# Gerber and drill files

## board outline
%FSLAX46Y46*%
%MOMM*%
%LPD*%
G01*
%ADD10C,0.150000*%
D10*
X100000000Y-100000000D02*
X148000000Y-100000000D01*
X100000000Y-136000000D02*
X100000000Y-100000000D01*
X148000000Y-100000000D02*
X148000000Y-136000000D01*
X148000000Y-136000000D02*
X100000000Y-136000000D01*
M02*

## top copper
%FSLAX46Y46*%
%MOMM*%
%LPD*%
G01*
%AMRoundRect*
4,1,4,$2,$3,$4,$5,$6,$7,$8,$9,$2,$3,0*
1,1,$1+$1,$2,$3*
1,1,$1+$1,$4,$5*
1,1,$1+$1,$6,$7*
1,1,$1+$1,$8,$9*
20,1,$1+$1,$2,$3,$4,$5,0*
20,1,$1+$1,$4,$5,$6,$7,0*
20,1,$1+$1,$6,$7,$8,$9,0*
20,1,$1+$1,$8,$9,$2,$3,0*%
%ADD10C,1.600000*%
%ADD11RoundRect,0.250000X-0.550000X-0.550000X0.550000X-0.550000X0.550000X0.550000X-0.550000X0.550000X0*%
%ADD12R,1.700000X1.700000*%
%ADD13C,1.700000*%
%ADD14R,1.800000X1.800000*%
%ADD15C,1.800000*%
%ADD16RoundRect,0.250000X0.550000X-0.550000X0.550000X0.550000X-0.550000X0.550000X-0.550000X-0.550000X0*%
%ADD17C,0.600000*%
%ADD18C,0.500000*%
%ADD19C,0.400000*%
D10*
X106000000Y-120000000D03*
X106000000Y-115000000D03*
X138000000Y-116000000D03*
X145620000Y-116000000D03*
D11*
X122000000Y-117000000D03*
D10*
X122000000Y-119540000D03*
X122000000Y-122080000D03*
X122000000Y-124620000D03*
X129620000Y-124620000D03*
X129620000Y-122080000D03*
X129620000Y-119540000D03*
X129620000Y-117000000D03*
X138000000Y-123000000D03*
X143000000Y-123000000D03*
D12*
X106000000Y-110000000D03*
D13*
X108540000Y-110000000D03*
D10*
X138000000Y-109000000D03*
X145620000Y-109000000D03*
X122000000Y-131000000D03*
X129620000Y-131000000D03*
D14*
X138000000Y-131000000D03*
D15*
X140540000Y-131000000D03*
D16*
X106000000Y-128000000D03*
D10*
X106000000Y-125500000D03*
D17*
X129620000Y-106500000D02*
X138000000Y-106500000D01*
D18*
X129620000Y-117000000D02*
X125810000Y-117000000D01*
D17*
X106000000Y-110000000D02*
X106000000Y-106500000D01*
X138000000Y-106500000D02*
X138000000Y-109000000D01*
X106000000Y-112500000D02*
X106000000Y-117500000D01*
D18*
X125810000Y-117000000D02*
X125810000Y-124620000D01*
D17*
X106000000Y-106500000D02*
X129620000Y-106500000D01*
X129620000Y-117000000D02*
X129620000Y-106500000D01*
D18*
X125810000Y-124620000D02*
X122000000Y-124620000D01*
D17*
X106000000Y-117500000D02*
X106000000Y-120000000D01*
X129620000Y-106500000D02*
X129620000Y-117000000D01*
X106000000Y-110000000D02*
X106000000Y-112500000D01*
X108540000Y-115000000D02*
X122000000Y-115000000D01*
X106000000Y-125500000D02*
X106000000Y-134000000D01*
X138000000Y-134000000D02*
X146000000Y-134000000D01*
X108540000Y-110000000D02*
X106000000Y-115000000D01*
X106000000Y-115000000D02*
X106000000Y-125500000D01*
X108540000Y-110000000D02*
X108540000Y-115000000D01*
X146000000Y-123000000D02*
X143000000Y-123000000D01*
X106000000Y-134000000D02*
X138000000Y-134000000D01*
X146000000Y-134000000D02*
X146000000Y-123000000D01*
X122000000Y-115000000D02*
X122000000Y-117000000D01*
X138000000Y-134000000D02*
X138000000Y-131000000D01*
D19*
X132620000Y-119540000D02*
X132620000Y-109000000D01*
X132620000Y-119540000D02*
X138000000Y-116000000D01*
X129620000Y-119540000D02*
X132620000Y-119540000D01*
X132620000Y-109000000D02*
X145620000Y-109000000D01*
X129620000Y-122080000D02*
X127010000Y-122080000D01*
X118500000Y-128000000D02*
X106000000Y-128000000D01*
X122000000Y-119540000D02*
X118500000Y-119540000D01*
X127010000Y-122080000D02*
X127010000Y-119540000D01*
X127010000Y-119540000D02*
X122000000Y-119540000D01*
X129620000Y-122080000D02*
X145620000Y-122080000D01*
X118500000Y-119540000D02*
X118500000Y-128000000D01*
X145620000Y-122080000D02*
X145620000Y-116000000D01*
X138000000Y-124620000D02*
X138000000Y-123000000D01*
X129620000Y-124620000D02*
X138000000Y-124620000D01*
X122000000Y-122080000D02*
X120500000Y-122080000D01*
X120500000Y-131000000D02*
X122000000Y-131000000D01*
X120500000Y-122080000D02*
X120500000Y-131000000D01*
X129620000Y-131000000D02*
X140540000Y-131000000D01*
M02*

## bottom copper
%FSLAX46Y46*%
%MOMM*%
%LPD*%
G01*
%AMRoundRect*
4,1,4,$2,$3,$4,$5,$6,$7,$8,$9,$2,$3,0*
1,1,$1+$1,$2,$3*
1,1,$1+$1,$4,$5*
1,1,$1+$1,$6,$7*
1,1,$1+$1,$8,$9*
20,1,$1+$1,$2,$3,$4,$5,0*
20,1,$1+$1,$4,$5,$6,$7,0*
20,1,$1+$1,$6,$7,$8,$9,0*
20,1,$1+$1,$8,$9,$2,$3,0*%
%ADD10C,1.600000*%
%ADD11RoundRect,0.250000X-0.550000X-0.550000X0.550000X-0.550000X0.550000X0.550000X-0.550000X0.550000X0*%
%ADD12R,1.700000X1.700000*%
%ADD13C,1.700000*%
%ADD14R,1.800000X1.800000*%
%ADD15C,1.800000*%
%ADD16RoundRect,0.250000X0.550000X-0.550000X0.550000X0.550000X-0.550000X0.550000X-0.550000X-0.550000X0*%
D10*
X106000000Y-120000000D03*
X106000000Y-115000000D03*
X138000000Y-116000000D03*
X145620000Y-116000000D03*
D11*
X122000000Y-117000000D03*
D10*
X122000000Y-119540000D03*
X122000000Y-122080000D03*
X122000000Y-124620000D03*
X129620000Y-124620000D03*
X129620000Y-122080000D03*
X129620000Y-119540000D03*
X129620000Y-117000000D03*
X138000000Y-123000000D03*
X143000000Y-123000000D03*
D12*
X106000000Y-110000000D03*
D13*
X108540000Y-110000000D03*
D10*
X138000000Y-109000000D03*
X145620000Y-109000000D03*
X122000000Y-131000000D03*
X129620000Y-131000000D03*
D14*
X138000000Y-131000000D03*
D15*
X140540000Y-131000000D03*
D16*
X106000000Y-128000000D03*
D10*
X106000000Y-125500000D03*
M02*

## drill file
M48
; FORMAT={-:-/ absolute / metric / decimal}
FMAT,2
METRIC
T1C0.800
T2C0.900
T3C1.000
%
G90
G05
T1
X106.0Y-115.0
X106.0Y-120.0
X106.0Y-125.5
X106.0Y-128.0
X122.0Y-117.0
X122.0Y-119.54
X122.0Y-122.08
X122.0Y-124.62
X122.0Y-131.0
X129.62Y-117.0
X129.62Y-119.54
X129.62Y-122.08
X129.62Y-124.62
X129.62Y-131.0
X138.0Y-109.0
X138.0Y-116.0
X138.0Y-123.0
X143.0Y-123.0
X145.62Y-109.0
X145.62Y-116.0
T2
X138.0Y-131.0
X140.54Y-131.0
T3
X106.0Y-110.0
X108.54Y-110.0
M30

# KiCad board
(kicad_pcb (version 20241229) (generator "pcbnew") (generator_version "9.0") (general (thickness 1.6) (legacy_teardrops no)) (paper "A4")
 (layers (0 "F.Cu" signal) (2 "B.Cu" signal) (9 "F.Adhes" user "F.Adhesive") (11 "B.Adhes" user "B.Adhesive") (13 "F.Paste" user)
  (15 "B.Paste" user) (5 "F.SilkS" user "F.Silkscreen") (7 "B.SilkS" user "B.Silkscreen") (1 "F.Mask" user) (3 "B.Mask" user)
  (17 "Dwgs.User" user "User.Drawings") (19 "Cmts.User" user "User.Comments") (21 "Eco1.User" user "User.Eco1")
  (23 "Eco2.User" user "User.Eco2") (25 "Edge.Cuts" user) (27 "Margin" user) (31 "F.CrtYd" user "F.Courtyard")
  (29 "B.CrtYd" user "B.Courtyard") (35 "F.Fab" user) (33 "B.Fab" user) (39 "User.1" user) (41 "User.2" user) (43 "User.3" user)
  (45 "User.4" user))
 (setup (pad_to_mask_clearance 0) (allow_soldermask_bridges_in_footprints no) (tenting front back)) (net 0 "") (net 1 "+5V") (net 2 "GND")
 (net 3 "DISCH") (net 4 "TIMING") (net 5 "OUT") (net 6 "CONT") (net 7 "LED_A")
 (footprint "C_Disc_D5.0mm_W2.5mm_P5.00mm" (layer "F.Cu") (at 106 120 90)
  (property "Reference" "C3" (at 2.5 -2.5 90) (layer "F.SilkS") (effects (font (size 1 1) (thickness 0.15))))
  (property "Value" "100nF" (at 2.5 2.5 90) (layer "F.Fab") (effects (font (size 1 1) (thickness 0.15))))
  (pad "1" thru_hole circle (at 0 0 90) (size 1.6 1.6) (drill 0.8) (layers "*.Cu" "*.Mask") (remove_unused_layers no) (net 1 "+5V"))
  (pad "2" thru_hole circle (at 5 0 90) (size 1.6 1.6) (drill 0.8) (layers "*.Cu" "*.Mask") (remove_unused_layers no) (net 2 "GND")))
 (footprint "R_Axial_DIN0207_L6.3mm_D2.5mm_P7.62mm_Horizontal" (layer "F.Cu") (at 138 116)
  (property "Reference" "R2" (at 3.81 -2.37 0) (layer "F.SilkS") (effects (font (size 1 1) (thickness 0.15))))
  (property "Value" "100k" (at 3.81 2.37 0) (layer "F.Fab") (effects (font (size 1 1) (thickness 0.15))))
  (pad "1" thru_hole circle (at 0 0) (size 1.6 1.6) (drill 0.8) (layers "*.Cu" "*.Mask") (remove_unused_layers no) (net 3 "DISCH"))
  (pad "2" thru_hole circle (at 7.62 0) (size 1.6 1.6) (drill 0.8) (layers "*.Cu" "*.Mask") (remove_unused_layers no) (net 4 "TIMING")))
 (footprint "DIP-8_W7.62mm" (layer "F.Cu") (at 122 117)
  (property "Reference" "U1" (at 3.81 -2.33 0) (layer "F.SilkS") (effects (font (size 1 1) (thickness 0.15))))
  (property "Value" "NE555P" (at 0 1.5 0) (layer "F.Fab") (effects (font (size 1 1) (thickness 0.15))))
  (pad "1" thru_hole roundrect (at 0 0) (size 1.6 1.6) (drill 0.8) (layers "*.Cu" "*.Mask") (remove_unused_layers no)
   (roundrect_rratio 0.15625) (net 2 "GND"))
  (pad "2" thru_hole circle (at 0 2.54) (size 1.6 1.6) (drill 0.8) (layers "*.Cu" "*.Mask") (remove_unused_layers no) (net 4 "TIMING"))
  (pad "3" thru_hole circle (at 0 5.08) (size 1.6 1.6) (drill 0.8) (layers "*.Cu" "*.Mask") (remove_unused_layers no) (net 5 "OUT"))
  (pad "4" thru_hole circle (at 0 7.62) (size 1.6 1.6) (drill 0.8) (layers "*.Cu" "*.Mask") (remove_unused_layers no) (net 1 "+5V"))
  (pad "5" thru_hole circle (at 7.62 7.62) (size 1.6 1.6) (drill 0.8) (layers "*.Cu" "*.Mask") (remove_unused_layers no) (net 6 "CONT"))
  (pad "6" thru_hole circle (at 7.62 5.08) (size 1.6 1.6) (drill 0.8) (layers "*.Cu" "*.Mask") (remove_unused_layers no) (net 4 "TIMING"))
  (pad "7" thru_hole circle (at 7.62 2.54) (size 1.6 1.6) (drill 0.8) (layers "*.Cu" "*.Mask") (remove_unused_layers no) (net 3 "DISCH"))
  (pad "8" thru_hole circle (at 7.62 0) (size 1.6 1.6) (drill 0.8) (layers "*.Cu" "*.Mask") (remove_unused_layers no) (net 1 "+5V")))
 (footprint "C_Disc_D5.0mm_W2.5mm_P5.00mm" (layer "F.Cu") (at 138 123)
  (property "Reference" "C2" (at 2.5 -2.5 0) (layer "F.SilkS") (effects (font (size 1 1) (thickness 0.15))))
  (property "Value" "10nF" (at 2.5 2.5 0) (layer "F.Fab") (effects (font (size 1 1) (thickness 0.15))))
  (pad "1" thru_hole circle (at 0 0) (size 1.6 1.6) (drill 0.8) (layers "*.Cu" "*.Mask") (remove_unused_layers no) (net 6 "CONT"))
  (pad "2" thru_hole circle (at 5 0) (size 1.6 1.6) (drill 0.8) (layers "*.Cu" "*.Mask") (remove_unused_layers no) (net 2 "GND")))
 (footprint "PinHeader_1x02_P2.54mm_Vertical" (layer "F.Cu") (at 106 110 90)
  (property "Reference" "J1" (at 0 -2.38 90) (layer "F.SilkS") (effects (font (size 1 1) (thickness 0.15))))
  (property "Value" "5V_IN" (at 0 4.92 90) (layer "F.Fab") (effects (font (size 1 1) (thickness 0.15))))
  (pad "1" thru_hole rect (at 0 0 90) (size 1.7 1.7) (drill 1) (layers "*.Cu" "*.Mask") (remove_unused_layers no) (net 1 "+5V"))
  (pad "2" thru_hole circle (at 0 2.54 90) (size 1.7 1.7) (drill 1) (layers "*.Cu" "*.Mask") (remove_unused_layers no) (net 2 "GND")))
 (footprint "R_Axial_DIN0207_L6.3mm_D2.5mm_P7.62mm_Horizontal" (layer "F.Cu") (at 138 109)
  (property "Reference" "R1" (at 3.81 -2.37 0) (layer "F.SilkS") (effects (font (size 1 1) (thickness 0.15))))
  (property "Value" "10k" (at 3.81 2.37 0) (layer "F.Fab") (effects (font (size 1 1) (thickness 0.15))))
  (pad "1" thru_hole circle (at 0 0) (size 1.6 1.6) (drill 0.8) (layers "*.Cu" "*.Mask") (remove_unused_layers no) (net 1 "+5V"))
  (pad "2" thru_hole circle (at 7.62 0) (size 1.6 1.6) (drill 0.8) (layers "*.Cu" "*.Mask") (remove_unused_layers no) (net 3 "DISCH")))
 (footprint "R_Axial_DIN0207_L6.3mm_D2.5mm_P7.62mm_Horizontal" (layer "F.Cu") (at 122 131)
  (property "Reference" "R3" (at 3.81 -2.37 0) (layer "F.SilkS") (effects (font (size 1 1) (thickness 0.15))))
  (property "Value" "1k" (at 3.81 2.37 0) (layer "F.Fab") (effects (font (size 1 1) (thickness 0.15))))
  (pad "1" thru_hole circle (at 0 0) (size 1.6 1.6) (drill 0.8) (layers "*.Cu" "*.Mask") (remove_unused_layers no) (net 5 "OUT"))
  (pad "2" thru_hole circle (at 7.62 0) (size 1.6 1.6) (drill 0.8) (layers "*.Cu" "*.Mask") (remove_unused_layers no) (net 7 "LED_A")))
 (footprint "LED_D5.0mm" (layer "F.Cu") (at 138 131)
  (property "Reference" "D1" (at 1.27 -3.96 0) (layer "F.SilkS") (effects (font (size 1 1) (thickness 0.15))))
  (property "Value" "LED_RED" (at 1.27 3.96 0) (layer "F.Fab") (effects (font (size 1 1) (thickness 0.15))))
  (pad "1" thru_hole rect (at 0 0) (size 1.8 1.8) (drill 0.9) (layers "*.Cu" "*.Mask") (remove_unused_layers no) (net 2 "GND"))
  (pad "2" thru_hole circle (at 2.54 0) (size 1.8 1.8) (drill 0.9) (layers "*.Cu" "*.Mask") (remove_unused_layers no) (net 7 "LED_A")))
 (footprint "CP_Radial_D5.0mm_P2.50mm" (layer "F.Cu") (at 106 128 90)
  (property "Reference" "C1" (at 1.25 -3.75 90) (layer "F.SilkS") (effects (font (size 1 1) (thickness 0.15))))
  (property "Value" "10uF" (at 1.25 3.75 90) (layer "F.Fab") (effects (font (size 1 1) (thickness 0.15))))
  (pad "1" thru_hole roundrect (at 0 0 90) (size 1.6 1.6) (drill 0.8) (layers "*.Cu" "*.Mask") (remove_unused_layers no)
   (roundrect_rratio 0.15625) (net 4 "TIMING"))
  (pad "2" thru_hole circle (at 2.5 0 90) (size 1.6 1.6) (drill 0.8) (layers "*.Cu" "*.Mask") (remove_unused_layers no) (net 2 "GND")))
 (gr_line (start 100 100) (end 148 100) (stroke (width 0.15) (type default)) (layer "Edge.Cuts"))
 (gr_line (start 100 136) (end 100 100) (stroke (width 0.15) (type default)) (layer "Edge.Cuts"))
 (gr_line (start 148 100) (end 148 136) (stroke (width 0.15) (type default)) (layer "Edge.Cuts"))
 (gr_line (start 148 136) (end 100 136) (stroke (width 0.15) (type default)) (layer "Edge.Cuts"))
 (segment (start 129.62 106.5) (end 138 106.5) (width 0.6) (layer "F.Cu") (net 1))
 (segment (start 129.62 117) (end 125.81 117) (width 0.5) (layer "F.Cu") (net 1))
 (segment (start 106 110) (end 106 106.5) (width 0.6) (layer "F.Cu") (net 1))
 (segment (start 138 106.5) (end 138 109) (width 0.6) (layer "F.Cu") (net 1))
 (segment (start 106 112.5) (end 106 117.5) (width 0.6) (layer "F.Cu") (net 1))
 (segment (start 125.81 117) (end 125.81 124.62) (width 0.5) (layer "F.Cu") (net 1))
 (segment (start 106 106.5) (end 129.62 106.5) (width 0.6) (layer "F.Cu") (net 1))
 (segment (start 129.62 117) (end 129.62 106.5) (width 0.6) (layer "F.Cu") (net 1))
 (segment (start 125.81 124.62) (end 122 124.62) (width 0.5) (layer "F.Cu") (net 1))
 (segment (start 106 117.5) (end 106 120) (width 0.6) (layer "F.Cu") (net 1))
 (segment (start 129.62 106.5) (end 129.62 117) (width 0.6) (layer "F.Cu") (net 1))
 (segment (start 106 110) (end 106 112.5) (width 0.6) (layer "F.Cu") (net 1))
 (segment (start 108.54 115) (end 122 115) (width 0.6) (layer "F.Cu") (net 2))
 (segment (start 106 125.5) (end 106 134) (width 0.6) (layer "F.Cu") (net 2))
 (segment (start 138 134) (end 146 134) (width 0.6) (layer "F.Cu") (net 2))
 (segment (start 108.54 110) (end 106 115) (width 0.6) (layer "F.Cu") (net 2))
 (segment (start 106 115) (end 106 125.5) (width 0.6) (layer "F.Cu") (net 2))
 (segment (start 108.54 110) (end 108.54 115) (width 0.6) (layer "F.Cu") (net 2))
 (segment (start 146 123) (end 143 123) (width 0.6) (layer "F.Cu") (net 2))
 (segment (start 106 134) (end 138 134) (width 0.6) (layer "F.Cu") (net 2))
 (segment (start 146 134) (end 146 123) (width 0.6) (layer "F.Cu") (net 2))
 (segment (start 122 115) (end 122 117) (width 0.6) (layer "F.Cu") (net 2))
 (segment (start 138 134) (end 138 131) (width 0.6) (layer "F.Cu") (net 2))
 (segment (start 132.62 119.54) (end 132.62 109) (width 0.4) (layer "F.Cu") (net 3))
 (segment (start 132.62 119.54) (end 138 116) (width 0.4) (layer "F.Cu") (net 3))
 (segment (start 129.62 119.54) (end 132.62 119.54) (width 0.4) (layer "F.Cu") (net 3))
 (segment (start 132.62 109) (end 145.62 109) (width 0.4) (layer "F.Cu") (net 3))
 (segment (start 129.62 122.08) (end 127.01 122.08) (width 0.4) (layer "F.Cu") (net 4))
 (segment (start 118.5 128) (end 106 128) (width 0.4) (layer "F.Cu") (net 4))
 (segment (start 122 119.54) (end 118.5 119.54) (width 0.4) (layer "F.Cu") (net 4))
 (segment (start 127.01 122.08) (end 127.01 119.54) (width 0.4) (layer "F.Cu") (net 4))
 (segment (start 127.01 119.54) (end 122 119.54) (width 0.4) (layer "F.Cu") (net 4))
 (segment (start 129.62 122.08) (end 145.62 122.08) (width 0.4) (layer "F.Cu") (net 4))
 (segment (start 118.5 119.54) (end 118.5 128) (width 0.4) (layer "F.Cu") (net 4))
 (segment (start 145.62 122.08) (end 145.62 116) (width 0.4) (layer "F.Cu") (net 4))
 (segment (start 138 124.62) (end 138 123) (width 0.4) (layer "F.Cu") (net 6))
 (segment (start 129.62 124.62) (end 138 124.62) (width 0.4) (layer "F.Cu") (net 6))
 (segment (start 122 122.08) (end 120.5 122.08) (width 0.4) (layer "F.Cu") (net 5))
 (segment (start 120.5 131) (end 122 131) (width 0.4) (layer "F.Cu") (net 5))
 (segment (start 120.5 122.08) (end 120.5 131) (width 0.4) (layer "F.Cu") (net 5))
 (segment (start 129.62 131) (end 140.54 131) (width 0.4) (layer "F.Cu") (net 7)))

